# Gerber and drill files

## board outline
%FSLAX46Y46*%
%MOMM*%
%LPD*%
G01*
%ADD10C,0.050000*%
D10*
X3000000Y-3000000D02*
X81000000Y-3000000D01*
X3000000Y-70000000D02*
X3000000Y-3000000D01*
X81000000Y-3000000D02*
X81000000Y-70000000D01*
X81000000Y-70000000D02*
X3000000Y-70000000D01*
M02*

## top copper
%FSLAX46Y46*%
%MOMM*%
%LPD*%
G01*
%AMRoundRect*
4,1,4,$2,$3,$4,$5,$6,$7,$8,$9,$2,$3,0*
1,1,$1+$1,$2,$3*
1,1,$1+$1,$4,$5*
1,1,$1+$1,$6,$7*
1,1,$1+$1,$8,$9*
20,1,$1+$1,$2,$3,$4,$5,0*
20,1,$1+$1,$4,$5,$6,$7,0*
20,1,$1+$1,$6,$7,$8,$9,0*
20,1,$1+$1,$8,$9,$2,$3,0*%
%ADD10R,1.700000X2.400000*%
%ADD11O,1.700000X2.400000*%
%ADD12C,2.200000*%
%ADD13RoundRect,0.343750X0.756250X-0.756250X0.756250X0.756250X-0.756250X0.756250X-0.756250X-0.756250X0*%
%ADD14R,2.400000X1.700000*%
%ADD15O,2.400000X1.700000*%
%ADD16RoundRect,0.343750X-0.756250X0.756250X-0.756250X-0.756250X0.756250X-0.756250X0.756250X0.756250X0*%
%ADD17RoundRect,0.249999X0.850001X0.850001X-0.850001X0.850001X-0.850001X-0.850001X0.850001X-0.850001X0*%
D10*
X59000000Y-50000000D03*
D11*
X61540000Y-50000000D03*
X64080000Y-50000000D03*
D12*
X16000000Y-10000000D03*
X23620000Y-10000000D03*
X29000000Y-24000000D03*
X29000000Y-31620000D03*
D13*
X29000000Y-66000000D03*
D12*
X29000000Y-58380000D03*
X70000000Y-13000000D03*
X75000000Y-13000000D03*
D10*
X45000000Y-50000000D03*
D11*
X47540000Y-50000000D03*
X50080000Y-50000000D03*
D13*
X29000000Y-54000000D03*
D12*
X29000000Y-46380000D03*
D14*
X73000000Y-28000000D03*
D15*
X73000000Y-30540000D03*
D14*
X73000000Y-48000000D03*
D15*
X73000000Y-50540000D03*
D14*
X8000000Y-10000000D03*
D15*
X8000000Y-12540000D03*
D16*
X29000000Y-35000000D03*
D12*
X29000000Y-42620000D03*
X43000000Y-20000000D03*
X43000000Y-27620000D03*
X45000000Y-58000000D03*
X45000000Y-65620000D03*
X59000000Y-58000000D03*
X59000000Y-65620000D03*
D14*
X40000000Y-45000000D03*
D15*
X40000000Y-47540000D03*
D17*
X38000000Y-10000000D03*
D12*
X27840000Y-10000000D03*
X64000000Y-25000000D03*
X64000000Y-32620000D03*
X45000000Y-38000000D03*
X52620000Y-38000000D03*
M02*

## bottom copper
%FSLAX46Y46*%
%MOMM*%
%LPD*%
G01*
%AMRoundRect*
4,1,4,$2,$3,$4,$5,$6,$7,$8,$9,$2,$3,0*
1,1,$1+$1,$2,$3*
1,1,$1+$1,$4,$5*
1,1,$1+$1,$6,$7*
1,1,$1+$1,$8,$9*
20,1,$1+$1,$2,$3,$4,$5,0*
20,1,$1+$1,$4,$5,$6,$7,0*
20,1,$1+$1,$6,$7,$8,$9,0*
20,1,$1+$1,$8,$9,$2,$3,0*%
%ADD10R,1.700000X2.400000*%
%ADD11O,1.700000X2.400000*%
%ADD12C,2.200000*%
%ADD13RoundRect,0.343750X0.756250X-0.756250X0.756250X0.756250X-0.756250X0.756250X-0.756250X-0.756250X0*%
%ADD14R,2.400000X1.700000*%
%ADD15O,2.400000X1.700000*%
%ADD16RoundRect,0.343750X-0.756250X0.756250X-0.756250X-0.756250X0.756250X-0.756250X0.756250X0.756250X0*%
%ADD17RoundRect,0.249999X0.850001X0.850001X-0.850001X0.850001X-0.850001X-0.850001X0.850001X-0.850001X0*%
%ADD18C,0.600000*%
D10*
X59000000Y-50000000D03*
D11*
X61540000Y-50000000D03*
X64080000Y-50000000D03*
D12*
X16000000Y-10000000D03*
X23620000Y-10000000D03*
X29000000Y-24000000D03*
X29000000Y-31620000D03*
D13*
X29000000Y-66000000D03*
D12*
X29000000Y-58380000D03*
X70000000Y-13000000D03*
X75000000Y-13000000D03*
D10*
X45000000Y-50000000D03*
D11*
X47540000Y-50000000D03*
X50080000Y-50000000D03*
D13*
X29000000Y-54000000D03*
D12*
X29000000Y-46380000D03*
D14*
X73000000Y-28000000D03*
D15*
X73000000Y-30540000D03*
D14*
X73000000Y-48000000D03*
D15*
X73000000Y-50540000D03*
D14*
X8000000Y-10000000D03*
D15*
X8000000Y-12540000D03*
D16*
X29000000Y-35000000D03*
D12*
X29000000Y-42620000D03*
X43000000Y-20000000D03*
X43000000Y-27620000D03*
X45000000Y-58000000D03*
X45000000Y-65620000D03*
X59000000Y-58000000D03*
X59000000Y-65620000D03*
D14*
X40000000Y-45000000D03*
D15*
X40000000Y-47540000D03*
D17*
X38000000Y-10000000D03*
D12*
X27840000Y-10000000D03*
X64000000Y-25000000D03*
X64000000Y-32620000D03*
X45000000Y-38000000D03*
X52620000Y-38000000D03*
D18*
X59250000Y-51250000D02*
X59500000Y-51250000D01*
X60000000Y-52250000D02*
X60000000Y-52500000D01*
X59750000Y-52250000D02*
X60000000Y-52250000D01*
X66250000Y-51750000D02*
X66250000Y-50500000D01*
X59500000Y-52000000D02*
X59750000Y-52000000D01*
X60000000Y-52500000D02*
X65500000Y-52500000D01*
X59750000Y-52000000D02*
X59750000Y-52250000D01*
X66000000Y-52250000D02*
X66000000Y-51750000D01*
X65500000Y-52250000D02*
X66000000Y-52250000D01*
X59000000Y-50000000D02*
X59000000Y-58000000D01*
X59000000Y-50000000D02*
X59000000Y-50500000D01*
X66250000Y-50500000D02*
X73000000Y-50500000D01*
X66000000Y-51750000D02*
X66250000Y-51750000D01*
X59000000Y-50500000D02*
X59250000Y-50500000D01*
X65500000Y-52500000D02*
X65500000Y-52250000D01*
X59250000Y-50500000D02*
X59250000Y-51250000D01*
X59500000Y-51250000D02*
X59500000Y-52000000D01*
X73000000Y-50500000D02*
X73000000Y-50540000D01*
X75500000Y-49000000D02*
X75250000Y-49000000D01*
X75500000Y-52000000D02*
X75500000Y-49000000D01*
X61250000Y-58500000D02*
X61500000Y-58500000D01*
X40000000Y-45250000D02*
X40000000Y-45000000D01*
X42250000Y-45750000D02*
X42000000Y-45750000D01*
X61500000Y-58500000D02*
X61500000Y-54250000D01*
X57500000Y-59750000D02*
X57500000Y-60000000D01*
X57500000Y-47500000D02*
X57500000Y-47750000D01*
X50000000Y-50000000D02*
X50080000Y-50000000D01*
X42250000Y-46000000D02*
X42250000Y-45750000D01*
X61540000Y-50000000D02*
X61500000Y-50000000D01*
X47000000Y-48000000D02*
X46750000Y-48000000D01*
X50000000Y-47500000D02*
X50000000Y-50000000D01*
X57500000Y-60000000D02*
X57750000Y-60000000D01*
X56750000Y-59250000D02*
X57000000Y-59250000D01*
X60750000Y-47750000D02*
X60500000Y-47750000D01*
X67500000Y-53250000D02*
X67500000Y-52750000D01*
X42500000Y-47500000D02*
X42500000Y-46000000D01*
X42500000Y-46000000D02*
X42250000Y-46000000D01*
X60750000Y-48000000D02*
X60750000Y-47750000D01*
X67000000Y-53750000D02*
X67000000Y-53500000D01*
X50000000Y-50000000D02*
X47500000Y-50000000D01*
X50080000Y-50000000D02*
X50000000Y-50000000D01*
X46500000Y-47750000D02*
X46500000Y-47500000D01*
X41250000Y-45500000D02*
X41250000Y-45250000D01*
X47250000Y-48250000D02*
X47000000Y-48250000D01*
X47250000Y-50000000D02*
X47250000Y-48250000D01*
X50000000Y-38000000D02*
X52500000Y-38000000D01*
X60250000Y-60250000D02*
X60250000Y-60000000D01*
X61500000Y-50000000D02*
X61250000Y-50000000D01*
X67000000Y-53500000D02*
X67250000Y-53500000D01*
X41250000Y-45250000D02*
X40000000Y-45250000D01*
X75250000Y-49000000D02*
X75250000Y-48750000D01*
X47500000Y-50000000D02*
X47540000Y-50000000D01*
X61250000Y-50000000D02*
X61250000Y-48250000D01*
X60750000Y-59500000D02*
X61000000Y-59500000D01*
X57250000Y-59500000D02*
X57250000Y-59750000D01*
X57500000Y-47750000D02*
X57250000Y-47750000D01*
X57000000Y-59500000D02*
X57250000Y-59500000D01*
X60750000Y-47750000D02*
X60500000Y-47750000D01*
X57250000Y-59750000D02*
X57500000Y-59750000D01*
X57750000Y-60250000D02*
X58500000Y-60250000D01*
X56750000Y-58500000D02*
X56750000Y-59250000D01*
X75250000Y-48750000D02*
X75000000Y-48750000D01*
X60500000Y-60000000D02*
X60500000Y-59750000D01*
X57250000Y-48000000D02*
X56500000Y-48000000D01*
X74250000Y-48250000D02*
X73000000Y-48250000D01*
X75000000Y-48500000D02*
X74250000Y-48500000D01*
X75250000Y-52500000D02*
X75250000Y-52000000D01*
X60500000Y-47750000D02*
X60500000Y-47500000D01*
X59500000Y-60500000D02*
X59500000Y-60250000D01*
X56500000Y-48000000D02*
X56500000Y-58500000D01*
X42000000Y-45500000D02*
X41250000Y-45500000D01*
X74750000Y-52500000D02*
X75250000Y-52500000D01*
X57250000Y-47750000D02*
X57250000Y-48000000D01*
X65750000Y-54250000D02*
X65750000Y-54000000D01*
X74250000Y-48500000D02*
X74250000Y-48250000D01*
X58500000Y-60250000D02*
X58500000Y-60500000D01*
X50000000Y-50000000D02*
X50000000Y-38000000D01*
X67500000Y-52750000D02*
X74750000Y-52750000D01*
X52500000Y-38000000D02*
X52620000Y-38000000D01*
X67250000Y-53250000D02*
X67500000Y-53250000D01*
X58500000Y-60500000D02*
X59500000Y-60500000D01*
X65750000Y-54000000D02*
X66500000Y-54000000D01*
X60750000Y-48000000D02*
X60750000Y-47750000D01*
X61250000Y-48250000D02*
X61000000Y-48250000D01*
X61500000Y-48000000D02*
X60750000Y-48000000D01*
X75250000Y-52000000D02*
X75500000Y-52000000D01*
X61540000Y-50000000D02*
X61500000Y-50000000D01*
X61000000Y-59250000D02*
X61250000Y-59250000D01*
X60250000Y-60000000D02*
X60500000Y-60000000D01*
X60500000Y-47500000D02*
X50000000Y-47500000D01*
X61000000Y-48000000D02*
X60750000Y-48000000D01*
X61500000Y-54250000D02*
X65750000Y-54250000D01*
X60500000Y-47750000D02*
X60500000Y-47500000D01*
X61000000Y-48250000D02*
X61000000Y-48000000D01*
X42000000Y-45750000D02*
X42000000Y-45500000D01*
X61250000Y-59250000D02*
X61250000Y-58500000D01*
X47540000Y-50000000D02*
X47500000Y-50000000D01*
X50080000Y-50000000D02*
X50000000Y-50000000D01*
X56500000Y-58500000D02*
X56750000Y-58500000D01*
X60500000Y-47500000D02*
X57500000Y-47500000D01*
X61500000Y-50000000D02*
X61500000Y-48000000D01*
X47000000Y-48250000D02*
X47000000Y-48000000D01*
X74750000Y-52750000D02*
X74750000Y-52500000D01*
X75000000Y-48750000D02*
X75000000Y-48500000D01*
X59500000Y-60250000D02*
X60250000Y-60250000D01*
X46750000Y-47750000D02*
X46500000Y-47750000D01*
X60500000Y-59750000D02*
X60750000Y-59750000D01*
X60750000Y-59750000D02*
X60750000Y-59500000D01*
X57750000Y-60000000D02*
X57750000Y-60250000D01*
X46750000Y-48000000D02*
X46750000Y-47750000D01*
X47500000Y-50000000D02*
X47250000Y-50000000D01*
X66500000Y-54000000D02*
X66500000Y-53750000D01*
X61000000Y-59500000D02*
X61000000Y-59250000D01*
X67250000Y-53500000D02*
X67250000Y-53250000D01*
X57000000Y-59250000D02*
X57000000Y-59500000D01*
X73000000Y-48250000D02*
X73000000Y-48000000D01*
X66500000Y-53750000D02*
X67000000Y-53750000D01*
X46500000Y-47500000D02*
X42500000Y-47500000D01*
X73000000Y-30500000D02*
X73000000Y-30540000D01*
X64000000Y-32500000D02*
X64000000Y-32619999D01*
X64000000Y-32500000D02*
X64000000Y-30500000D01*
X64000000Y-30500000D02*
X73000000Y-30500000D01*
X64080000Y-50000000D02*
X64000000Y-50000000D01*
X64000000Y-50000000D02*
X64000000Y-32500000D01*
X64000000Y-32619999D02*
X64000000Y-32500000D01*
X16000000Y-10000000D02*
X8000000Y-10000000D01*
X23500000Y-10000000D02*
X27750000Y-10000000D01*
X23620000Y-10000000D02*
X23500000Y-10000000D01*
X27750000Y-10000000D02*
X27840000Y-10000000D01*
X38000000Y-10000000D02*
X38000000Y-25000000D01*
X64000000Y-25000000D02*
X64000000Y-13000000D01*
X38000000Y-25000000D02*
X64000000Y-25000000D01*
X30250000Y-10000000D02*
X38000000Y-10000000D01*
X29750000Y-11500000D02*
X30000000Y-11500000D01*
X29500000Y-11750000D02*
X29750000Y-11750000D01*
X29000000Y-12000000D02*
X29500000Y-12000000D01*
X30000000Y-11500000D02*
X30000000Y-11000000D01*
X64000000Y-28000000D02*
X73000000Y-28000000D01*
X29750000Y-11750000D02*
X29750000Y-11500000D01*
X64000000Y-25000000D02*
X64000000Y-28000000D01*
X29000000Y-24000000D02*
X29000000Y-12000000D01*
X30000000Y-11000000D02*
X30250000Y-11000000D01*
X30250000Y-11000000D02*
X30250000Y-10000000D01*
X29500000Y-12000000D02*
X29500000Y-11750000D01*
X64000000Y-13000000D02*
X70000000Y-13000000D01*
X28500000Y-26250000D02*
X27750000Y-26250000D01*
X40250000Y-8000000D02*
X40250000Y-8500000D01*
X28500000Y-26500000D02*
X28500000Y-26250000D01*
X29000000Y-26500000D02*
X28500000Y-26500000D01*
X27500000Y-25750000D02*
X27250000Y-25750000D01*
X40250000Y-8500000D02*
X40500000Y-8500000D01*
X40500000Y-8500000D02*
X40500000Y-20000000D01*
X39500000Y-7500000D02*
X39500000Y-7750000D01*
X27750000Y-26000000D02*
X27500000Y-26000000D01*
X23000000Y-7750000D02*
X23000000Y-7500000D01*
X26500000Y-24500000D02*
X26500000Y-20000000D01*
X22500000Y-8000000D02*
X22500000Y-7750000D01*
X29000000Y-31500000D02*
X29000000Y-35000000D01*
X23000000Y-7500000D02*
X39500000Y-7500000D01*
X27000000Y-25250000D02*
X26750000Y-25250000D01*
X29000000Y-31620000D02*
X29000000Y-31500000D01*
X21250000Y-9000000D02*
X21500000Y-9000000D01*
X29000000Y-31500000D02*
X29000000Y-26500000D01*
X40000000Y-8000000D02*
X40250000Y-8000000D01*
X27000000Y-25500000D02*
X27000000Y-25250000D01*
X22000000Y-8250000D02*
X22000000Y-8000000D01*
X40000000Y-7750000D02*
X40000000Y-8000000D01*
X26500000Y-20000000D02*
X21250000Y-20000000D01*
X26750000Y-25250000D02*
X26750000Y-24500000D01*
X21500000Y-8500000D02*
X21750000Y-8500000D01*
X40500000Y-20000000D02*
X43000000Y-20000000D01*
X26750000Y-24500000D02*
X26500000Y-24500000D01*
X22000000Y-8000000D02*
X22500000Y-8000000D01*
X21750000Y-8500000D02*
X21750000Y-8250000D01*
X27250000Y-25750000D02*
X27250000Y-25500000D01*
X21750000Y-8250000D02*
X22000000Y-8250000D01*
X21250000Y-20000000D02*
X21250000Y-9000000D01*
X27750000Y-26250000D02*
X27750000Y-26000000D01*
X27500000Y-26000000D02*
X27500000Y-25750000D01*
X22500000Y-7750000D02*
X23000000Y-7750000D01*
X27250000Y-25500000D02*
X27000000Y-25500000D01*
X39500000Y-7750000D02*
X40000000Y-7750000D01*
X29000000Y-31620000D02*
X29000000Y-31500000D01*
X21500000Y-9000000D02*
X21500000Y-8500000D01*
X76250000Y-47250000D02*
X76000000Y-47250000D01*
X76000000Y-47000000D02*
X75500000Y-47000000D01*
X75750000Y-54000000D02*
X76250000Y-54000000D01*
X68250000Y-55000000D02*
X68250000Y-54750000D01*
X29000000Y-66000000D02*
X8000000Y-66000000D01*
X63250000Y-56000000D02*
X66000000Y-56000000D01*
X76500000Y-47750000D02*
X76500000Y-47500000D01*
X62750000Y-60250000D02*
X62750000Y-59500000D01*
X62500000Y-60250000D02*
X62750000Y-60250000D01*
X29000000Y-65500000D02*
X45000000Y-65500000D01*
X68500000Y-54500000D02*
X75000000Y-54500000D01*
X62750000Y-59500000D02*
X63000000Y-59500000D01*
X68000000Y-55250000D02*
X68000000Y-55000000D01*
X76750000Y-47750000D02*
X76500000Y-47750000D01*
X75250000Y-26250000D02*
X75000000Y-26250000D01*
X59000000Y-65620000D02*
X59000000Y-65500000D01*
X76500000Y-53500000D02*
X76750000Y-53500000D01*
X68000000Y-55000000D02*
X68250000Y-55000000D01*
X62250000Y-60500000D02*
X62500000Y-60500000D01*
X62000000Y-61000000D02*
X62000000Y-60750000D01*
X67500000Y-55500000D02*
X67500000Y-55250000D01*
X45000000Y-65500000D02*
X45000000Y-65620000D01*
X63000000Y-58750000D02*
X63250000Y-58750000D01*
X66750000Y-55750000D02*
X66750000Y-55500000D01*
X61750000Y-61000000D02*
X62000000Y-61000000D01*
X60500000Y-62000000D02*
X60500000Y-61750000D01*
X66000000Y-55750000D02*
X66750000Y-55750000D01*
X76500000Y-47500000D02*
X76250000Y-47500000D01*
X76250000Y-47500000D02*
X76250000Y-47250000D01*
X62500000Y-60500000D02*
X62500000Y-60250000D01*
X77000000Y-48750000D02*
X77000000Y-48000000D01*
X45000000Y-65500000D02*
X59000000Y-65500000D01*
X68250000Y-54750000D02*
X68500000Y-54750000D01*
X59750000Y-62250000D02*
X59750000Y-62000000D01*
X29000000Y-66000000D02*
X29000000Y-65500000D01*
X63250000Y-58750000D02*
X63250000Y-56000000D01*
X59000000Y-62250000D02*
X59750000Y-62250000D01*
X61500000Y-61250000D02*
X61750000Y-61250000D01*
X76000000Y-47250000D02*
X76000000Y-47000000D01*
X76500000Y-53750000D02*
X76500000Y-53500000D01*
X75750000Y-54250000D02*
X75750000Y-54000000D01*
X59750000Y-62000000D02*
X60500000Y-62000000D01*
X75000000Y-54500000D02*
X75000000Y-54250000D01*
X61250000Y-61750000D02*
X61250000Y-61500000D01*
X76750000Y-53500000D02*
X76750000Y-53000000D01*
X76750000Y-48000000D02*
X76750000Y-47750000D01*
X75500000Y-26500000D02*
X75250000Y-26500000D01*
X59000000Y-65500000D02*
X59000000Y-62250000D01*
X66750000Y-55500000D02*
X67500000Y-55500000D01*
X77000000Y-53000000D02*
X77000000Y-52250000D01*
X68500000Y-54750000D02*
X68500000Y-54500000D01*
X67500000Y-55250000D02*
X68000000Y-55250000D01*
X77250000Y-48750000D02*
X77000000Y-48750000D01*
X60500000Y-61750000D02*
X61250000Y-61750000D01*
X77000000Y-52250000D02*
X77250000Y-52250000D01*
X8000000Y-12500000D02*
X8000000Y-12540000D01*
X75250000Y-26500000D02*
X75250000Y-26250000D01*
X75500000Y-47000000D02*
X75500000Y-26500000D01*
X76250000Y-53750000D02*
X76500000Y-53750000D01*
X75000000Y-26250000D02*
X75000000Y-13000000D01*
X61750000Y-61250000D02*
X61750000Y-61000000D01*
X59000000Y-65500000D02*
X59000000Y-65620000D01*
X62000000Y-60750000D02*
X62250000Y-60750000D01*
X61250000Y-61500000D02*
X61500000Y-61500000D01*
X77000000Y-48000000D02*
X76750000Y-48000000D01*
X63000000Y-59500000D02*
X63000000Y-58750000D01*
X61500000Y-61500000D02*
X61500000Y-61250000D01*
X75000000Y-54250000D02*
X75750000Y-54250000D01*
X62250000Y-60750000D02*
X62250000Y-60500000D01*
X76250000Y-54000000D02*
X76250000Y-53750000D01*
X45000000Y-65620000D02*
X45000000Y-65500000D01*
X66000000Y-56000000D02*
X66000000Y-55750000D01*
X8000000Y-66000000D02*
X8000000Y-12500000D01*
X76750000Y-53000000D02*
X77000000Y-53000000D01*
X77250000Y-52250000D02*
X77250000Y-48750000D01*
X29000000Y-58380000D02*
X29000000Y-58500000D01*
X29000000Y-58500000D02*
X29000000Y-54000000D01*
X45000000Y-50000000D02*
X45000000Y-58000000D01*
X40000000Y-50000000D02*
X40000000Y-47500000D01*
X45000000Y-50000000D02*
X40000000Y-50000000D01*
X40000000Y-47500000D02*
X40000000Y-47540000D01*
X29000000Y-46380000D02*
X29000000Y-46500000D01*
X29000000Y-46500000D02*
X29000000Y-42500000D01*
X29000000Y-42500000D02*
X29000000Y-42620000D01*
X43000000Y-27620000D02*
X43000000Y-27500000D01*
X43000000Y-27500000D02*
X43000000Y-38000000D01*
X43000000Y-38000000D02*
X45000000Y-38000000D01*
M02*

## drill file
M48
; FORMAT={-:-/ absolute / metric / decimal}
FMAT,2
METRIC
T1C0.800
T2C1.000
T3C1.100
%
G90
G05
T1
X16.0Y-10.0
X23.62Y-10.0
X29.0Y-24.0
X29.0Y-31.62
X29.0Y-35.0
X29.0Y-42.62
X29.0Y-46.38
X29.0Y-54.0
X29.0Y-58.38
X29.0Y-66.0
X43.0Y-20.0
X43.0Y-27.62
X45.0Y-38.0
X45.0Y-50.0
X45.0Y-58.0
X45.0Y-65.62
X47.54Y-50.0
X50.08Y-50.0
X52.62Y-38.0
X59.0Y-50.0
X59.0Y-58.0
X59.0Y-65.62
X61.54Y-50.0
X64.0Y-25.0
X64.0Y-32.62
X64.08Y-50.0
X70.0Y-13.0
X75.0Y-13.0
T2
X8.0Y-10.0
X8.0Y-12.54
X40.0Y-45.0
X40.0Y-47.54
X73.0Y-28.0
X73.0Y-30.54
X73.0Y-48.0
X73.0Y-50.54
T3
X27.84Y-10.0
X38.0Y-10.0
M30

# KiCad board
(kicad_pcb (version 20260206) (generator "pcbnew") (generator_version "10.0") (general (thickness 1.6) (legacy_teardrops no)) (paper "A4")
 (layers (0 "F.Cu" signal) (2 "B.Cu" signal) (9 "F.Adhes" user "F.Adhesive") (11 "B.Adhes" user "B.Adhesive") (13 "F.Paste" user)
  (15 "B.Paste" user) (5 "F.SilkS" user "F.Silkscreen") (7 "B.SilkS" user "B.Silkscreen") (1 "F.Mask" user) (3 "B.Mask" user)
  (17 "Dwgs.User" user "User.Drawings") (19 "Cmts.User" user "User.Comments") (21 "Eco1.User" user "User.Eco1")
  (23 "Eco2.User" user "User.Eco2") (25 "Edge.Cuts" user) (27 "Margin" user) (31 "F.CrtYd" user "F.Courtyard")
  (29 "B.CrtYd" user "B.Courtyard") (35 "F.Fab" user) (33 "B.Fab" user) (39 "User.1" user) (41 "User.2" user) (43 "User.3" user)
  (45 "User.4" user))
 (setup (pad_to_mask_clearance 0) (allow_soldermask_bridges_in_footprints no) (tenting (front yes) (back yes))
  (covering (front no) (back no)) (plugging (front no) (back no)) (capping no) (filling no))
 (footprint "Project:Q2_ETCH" (layer "F.Cu") (at 59 50)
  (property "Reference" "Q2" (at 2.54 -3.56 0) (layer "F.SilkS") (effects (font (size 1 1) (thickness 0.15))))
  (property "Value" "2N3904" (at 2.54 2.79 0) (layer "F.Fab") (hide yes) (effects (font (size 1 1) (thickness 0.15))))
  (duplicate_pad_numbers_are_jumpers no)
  (pad "1" thru_hole rect (at 0 0) (size 1.7 2.4) (drill 0.8) (layers "*.Cu" "*.Mask") (remove_unused_layers no) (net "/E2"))
  (pad "2" thru_hole oval (at 2.54 0) (size 1.7 2.4) (drill 0.8) (layers "*.Cu" "*.Mask") (remove_unused_layers no) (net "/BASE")
   (thermal_bridge_angle 45))
  (pad "3" thru_hole oval (at 5.08 0) (size 1.7 2.4) (drill 0.8) (layers "*.Cu" "*.Mask") (remove_unused_layers no) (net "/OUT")
   (thermal_bridge_angle 45)))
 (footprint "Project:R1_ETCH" (layer "F.Cu") (at 16 10)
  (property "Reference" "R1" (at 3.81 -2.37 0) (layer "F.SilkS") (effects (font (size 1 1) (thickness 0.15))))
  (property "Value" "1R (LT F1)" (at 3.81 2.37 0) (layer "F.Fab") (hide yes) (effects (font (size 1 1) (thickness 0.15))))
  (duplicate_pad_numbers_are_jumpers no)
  (pad "1" thru_hole circle (at 0 0) (size 2.2 2.2) (drill 0.8) (layers "*.Cu" "*.Mask") (remove_unused_layers no) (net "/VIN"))
  (pad "2" thru_hole circle (at 7.62 0) (size 2.2 2.2) (drill 0.8) (layers "*.Cu" "*.Mask") (remove_unused_layers no) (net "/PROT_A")))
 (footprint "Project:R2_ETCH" (layer "F.Cu") (at 29 24 -90)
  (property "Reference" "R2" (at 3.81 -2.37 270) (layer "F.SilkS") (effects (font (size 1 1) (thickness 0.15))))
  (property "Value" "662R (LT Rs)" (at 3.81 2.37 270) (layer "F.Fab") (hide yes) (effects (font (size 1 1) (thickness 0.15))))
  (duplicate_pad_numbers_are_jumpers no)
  (pad "1" thru_hole circle (at 0 0 270) (size 2.2 2.2) (drill 0.8) (layers "*.Cu" "*.Mask") (remove_unused_layers no) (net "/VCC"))
  (pad "2" thru_hole circle (at 7.62 0 270) (size 2.2 2.2) (drill 0.8) (layers "*.Cu" "*.Mask") (remove_unused_layers no) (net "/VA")))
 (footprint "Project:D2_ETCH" (layer "F.Cu") (at 29 66 90)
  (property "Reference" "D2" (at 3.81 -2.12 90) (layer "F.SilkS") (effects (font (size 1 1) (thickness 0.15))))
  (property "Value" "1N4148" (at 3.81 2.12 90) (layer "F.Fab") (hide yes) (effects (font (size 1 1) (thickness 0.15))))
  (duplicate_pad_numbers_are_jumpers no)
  (pad "1" thru_hole roundrect (at 0 0 90) (size 2.2 2.2) (drill 0.8) (layers "*.Cu" "*.Mask") (remove_unused_layers no)
   (roundrect_rratio 0.15625) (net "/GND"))
  (pad "2" thru_hole circle (at 7.62 0 90) (size 2.2 2.2) (drill 0.8) (layers "*.Cu" "*.Mask") (remove_unused_layers no) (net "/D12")))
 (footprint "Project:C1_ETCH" (layer "F.Cu") (at 70 13)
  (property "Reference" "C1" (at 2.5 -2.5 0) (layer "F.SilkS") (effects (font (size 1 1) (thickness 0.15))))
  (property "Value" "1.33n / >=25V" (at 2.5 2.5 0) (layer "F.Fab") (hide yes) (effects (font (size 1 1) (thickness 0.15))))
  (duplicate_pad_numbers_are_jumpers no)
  (pad "1" thru_hole circle (at 0 0) (size 2.2 2.2) (drill 0.8) (layers "*.Cu" "*.Mask") (remove_unused_layers no) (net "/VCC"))
  (pad "2" thru_hole circle (at 5 0) (size 2.2 2.2) (drill 0.8) (layers "*.Cu" "*.Mask") (remove_unused_layers no) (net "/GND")))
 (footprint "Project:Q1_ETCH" (layer "F.Cu") (at 45 50)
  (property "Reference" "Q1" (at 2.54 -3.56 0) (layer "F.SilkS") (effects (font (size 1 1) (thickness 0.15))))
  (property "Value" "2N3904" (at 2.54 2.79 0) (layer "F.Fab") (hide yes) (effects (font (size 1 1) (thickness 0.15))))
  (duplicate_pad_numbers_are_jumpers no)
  (pad "1" thru_hole rect (at 0 0) (size 1.7 2.4) (drill 0.8) (layers "*.Cu" "*.Mask") (remove_unused_layers no) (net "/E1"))
  (pad "2" thru_hole oval (at 2.54 0) (size 1.7 2.4) (drill 0.8) (layers "*.Cu" "*.Mask") (remove_unused_layers no) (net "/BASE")
   (thermal_bridge_angle 45))
  (pad "3" thru_hole oval (at 5.08 0) (size 1.7 2.4) (drill 0.8) (layers "*.Cu" "*.Mask") (remove_unused_layers no) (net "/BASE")
   (thermal_bridge_angle 45)))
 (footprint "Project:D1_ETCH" (layer "F.Cu") (at 29 54 90)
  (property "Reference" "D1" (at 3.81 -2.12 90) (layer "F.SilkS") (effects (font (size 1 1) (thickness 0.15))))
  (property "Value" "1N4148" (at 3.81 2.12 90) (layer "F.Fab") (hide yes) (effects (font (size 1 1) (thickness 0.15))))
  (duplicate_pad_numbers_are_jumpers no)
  (pad "1" thru_hole roundrect (at 0 0 90) (size 2.2 2.2) (drill 0.8) (layers "*.Cu" "*.Mask") (remove_unused_layers no)
   (roundrect_rratio 0.15625) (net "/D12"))
  (pad "2" thru_hole circle (at 7.62 0 90) (size 2.2 2.2) (drill 0.8) (layers "*.Cu" "*.Mask") (remove_unused_layers no) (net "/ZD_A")))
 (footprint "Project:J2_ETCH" (layer "F.Cu") (at 73 28)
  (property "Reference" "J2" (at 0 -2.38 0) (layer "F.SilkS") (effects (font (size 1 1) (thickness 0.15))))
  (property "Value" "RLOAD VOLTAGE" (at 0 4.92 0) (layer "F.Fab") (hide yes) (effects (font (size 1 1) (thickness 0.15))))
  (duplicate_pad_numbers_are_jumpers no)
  (pad "1" thru_hole rect (at 0 0) (size 2.4 1.7) (drill 1) (layers "*.Cu" "*.Mask") (remove_unused_layers no) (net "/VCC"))
  (pad "2" thru_hole oval (at 0 2.54) (size 2.4 1.7) (drill 1) (layers "*.Cu" "*.Mask") (remove_unused_layers no) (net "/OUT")
   (thermal_bridge_angle 45)))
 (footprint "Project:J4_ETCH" (layer "F.Cu") (at 73 48)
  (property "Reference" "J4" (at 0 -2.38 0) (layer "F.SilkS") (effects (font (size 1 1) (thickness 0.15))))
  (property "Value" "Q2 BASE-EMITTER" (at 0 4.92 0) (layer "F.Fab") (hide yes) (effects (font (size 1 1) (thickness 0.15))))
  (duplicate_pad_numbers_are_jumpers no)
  (pad "1" thru_hole rect (at 0 0) (size 2.4 1.7) (drill 1) (layers "*.Cu" "*.Mask") (remove_unused_layers no) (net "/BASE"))
  (pad "2" thru_hole oval (at 0 2.54) (size 2.4 1.7) (drill 1) (layers "*.Cu" "*.Mask") (remove_unused_layers no) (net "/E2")
   (thermal_bridge_angle 45)))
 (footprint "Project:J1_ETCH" (layer "F.Cu") (at 8 10)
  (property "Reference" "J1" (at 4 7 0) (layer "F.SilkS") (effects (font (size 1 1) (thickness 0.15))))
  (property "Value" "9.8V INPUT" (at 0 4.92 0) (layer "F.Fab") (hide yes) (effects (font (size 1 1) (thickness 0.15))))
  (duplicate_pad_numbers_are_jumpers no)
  (pad "1" thru_hole rect (at 0 0) (size 2.4 1.7) (drill 1) (layers "*.Cu" "*.Mask") (remove_unused_layers no) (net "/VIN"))
  (pad "2" thru_hole oval (at 0 2.54) (size 2.4 1.7) (drill 1) (layers "*.Cu" "*.Mask") (remove_unused_layers no) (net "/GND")
   (thermal_bridge_angle 45)))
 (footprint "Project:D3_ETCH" (layer "F.Cu") (at 29 35 -90)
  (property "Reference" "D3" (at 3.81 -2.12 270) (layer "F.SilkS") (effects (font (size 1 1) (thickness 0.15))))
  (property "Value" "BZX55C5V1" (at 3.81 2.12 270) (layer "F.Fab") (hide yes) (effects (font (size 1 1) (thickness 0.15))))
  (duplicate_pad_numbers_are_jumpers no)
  (pad "1" thru_hole roundrect (at 0 0 270) (size 2.2 2.2) (drill 0.8) (layers "*.Cu" "*.Mask") (remove_unused_layers no)
   (roundrect_rratio 0.15625) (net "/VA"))
  (pad "2" thru_hole circle (at 7.62 0 270) (size 2.2 2.2) (drill 0.8) (layers "*.Cu" "*.Mask") (remove_unused_layers no) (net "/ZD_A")))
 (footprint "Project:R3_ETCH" (layer "F.Cu") (at 43 20 -90)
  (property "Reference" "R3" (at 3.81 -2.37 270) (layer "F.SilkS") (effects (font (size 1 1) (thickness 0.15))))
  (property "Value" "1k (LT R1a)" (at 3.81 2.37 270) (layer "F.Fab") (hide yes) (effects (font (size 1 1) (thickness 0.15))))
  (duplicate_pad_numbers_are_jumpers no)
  (pad "1" thru_hole circle (at 0 0 270) (size 2.2 2.2) (drill 0.8) (layers "*.Cu" "*.Mask") (remove_unused_layers no) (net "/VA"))
  (pad "2" thru_hole circle (at 7.62 0 270) (size 2.2 2.2) (drill 0.8) (layers "*.Cu" "*.Mask") (remove_unused_layers no) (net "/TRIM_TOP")))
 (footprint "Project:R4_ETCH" (layer "F.Cu") (at 45 58 -90)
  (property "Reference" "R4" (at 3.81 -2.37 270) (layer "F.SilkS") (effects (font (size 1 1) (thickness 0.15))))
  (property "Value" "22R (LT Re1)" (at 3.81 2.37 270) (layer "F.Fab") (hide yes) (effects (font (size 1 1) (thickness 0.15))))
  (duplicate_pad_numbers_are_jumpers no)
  (pad "1" thru_hole circle (at 0 0 270) (size 2.2 2.2) (drill 0.8) (layers "*.Cu" "*.Mask") (remove_unused_layers no) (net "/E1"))
  (pad "2" thru_hole circle (at 7.62 0 270) (size 2.2 2.2) (drill 0.8) (layers "*.Cu" "*.Mask") (remove_unused_layers no) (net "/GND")))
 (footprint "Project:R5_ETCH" (layer "F.Cu") (at 59 58 -90)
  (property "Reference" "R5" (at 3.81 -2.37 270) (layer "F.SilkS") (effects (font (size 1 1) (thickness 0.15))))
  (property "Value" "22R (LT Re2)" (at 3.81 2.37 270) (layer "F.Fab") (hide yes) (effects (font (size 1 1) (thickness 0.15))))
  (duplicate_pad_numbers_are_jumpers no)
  (pad "1" thru_hole circle (at 0 0 270) (size 2.2 2.2) (drill 0.8) (layers "*.Cu" "*.Mask") (remove_unused_layers no) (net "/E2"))
  (pad "2" thru_hole circle (at 7.62 0 270) (size 2.2 2.2) (drill 0.8) (layers "*.Cu" "*.Mask") (remove_unused_layers no) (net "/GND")))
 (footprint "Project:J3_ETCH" (layer "F.Cu") (at 40 45)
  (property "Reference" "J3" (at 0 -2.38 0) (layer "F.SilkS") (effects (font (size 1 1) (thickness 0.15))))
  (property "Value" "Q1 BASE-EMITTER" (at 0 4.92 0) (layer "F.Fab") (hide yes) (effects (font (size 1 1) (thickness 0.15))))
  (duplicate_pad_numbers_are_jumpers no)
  (pad "1" thru_hole rect (at 0 0) (size 2.4 1.7) (drill 1) (layers "*.Cu" "*.Mask") (remove_unused_layers no) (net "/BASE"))
  (pad "2" thru_hole oval (at 0 2.54) (size 2.4 1.7) (drill 1) (layers "*.Cu" "*.Mask") (remove_unused_layers no) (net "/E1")
   (thermal_bridge_angle 45)))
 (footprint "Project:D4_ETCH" (layer "F.Cu") (at 38 10 180)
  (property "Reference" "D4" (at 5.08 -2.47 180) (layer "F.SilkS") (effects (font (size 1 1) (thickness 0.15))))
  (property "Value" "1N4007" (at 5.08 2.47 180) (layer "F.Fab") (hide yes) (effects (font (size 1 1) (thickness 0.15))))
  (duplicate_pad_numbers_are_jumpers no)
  (pad "1" thru_hole roundrect (at 0 0 180) (size 2.2 2.2) (drill 1.1) (layers "*.Cu" "*.Mask") (remove_unused_layers no)
   (roundrect_rratio 0.113636) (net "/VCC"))
  (pad "2" thru_hole circle (at 10.16 0 180) (size 2.2 2.2) (drill 1.1) (layers "*.Cu" "*.Mask") (remove_unused_layers no) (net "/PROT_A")))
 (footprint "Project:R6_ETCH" (layer "F.Cu") (at 64 25 -90)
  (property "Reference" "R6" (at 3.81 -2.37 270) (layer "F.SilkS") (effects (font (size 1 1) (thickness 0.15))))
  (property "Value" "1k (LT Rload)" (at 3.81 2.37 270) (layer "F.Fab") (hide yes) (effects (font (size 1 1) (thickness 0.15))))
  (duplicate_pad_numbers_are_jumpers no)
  (pad "1" thru_hole circle (at 0 0 270) (size 2.2 2.2) (drill 0.8) (layers "*.Cu" "*.Mask") (remove_unused_layers no) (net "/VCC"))
  (pad "2" thru_hole circle (at 7.62 0 270) (size 2.2 2.2) (drill 0.8) (layers "*.Cu" "*.Mask") (remove_unused_layers no) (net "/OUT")))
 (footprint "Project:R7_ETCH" (layer "F.Cu") (at 45 38)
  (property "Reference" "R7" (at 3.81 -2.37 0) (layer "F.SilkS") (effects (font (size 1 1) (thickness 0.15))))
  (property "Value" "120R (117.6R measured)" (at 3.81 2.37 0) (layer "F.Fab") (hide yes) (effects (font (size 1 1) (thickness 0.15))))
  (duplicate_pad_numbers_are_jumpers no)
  (pad "1" thru_hole circle (at 0 0) (size 2.2 2.2) (drill 0.8) (layers "*.Cu" "*.Mask") (remove_unused_layers no) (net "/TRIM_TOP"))
  (pad "2" thru_hole circle (at 7.62 0) (size 2.2 2.2) (drill 0.8) (layers "*.Cu" "*.Mask") (remove_unused_layers no) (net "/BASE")))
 (gr_line (start 3 3) (end 81 3) (stroke (width 0.05) (type default)) (layer "Edge.Cuts"))
 (gr_line (start 3 70) (end 3 3) (stroke (width 0.05) (type default)) (layer "Edge.Cuts"))
 (gr_line (start 81 3) (end 81 70) (stroke (width 0.05) (type default)) (layer "Edge.Cuts"))
 (gr_line (start 81 70) (end 3 70) (stroke (width 0.05) (type default)) (layer "Edge.Cuts"))
 (segment (start 59.25 51.25) (end 59.5 51.25) (width 0.6) (layer "B.Cu") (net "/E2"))
 (segment (start 60 52.25) (end 60 52.5) (width 0.6) (layer "B.Cu") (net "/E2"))
 (segment (start 59.75 52.25) (end 60 52.25) (width 0.6) (layer "B.Cu") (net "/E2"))
 (segment (start 66.25 51.75) (end 66.25 50.5) (width 0.6) (layer "B.Cu") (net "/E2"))
 (segment (start 59.5 52) (end 59.75 52) (width 0.6) (layer "B.Cu") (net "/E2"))
 (segment (start 60 52.5) (end 65.5 52.5) (width 0.6) (layer "B.Cu") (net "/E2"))
 (segment (start 59.75 52) (end 59.75 52.25) (width 0.6) (layer "B.Cu") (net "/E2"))
 (segment (start 66 52.25) (end 66 51.75) (width 0.6) (layer "B.Cu") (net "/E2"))
 (segment (start 65.5 52.25) (end 66 52.25) (width 0.6) (layer "B.Cu") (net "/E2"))
 (segment (start 59 50) (end 59 58) (width 0.6) (layer "B.Cu") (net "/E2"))
 (segment (start 59 50) (end 59 50.5) (width 0.6) (layer "B.Cu") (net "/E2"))
 (segment (start 66.25 50.5) (end 73 50.5) (width 0.6) (layer "B.Cu") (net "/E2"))
 (segment (start 66 51.75) (end 66.25 51.75) (width 0.6) (layer "B.Cu") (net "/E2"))
 (segment (start 59 50.5) (end 59.25 50.5) (width 0.6) (layer "B.Cu") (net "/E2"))
 (segment (start 65.5 52.5) (end 65.5 52.25) (width 0.6) (layer "B.Cu") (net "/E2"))
 (segment (start 59.25 50.5) (end 59.25 51.25) (width 0.6) (layer "B.Cu") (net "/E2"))
 (segment (start 59.5 51.25) (end 59.5 52) (width 0.6) (layer "B.Cu") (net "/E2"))
 (segment (start 73 50.5) (end 73 50.54) (width 0.6) (layer "B.Cu") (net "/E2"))
 (segment (start 75.5 49) (end 75.25 49) (width 0.6) (layer "B.Cu") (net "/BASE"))
 (segment (start 75.5 52) (end 75.5 49) (width 0.6) (layer "B.Cu") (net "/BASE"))
 (segment (start 61.25 58.5) (end 61.5 58.5) (width 0.6) (layer "B.Cu") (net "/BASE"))
 (segment (start 40 45.25) (end 40 45) (width 0.6) (layer "B.Cu") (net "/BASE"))
 (segment (start 42.25 45.75) (end 42 45.75) (width 0.6) (layer "B.Cu") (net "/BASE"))
 (segment (start 61.5 58.5) (end 61.5 54.25) (width 0.6) (layer "B.Cu") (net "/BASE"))
 (segment (start 57.5 59.75) (end 57.5 60) (width 0.6) (layer "B.Cu") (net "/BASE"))
 (segment (start 57.5 47.5) (end 57.5 47.75) (width 0.6) (layer "B.Cu") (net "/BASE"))
 (segment (start 50 50) (end 50.08 50) (width 0.6) (layer "B.Cu") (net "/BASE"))
 (segment (start 42.25 46) (end 42.25 45.75) (width 0.6) (layer "B.Cu") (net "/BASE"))
 (segment (start 61.54 50) (end 61.5 50) (width 0.6) (layer "B.Cu") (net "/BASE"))
 (segment (start 47 48) (end 46.75 48) (width 0.6) (layer "B.Cu") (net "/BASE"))
 (segment (start 50 47.5) (end 50 50) (width 0.6) (layer "B.Cu") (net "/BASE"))
 (segment (start 57.5 60) (end 57.75 60) (width 0.6) (layer "B.Cu") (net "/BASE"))
 (segment (start 56.75 59.25) (end 57 59.25) (width 0.6) (layer "B.Cu") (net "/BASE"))
 (segment (start 60.75 47.75) (end 60.5 47.75) (width 0.6) (layer "B.Cu") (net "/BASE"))
 (segment (start 67.5 53.25) (end 67.5 52.75) (width 0.6) (layer "B.Cu") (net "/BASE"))
 (segment (start 42.5 47.5) (end 42.5 46) (width 0.6) (layer "B.Cu") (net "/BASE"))
 (segment (start 42.5 46) (end 42.25 46) (width 0.6) (layer "B.Cu") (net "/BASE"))
 (segment (start 60.75 48) (end 60.75 47.75) (width 0.6) (layer "B.Cu") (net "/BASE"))
 (segment (start 67 53.75) (end 67 53.5) (width 0.6) (layer "B.Cu") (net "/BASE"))
 (segment (start 50 50) (end 47.5 50) (width 0.6) (layer "B.Cu") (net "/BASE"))
 (segment (start 50.08 50) (end 50 50) (width 0.6) (layer "B.Cu") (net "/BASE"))
 (segment (start 46.5 47.75) (end 46.5 47.5) (width 0.6) (layer "B.Cu") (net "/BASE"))
 (segment (start 41.25 45.5) (end 41.25 45.25) (width 0.6) (layer "B.Cu") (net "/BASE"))
 (segment (start 47.25 48.25) (end 47 48.25) (width 0.6) (layer "B.Cu") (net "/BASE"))
 (segment (start 47.25 50) (end 47.25 48.25) (width 0.6) (layer "B.Cu") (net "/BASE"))
 (segment (start 50 38) (end 52.5 38) (width 0.6) (layer "B.Cu") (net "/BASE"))
 (segment (start 60.25 60.25) (end 60.25 60) (width 0.6) (layer "B.Cu") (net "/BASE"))
 (segment (start 61.5 50) (end 61.25 50) (width 0.6) (layer "B.Cu") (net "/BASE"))
 (segment (start 67 53.5) (end 67.25 53.5) (width 0.6) (layer "B.Cu") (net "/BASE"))
 (segment (start 41.25 45.25) (end 40 45.25) (width 0.6) (layer "B.Cu") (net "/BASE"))
 (segment (start 75.25 49) (end 75.25 48.75) (width 0.6) (layer "B.Cu") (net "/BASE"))
 (segment (start 47.5 50) (end 47.54 50) (width 0.6) (layer "B.Cu") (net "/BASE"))
 (segment (start 61.25 50) (end 61.25 48.25) (width 0.6) (layer "B.Cu") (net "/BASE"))
 (segment (start 60.75 59.5) (end 61 59.5) (width 0.6) (layer "B.Cu") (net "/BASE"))
 (segment (start 57.25 59.5) (end 57.25 59.75) (width 0.6) (layer "B.Cu") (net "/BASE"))
 (segment (start 57.5 47.75) (end 57.25 47.75) (width 0.6) (layer "B.Cu") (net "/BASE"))
 (segment (start 57 59.5) (end 57.25 59.5) (width 0.6) (layer "B.Cu") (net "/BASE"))
 (segment (start 60.75 47.75) (end 60.5 47.75) (width 0.6) (layer "B.Cu") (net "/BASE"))
 (segment (start 57.25 59.75) (end 57.5 59.75) (width 0.6) (layer "B.Cu") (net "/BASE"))
 (segment (start 57.75 60.25) (end 58.5 60.25) (width 0.6) (layer "B.Cu") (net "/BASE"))
 (segment (start 56.75 58.5) (end 56.75 59.25) (width 0.6) (layer "B.Cu") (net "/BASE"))
 (segment (start 75.25 48.75) (end 75 48.75) (width 0.6) (layer "B.Cu") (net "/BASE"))
 (segment (start 60.5 60) (end 60.5 59.75) (width 0.6) (layer "B.Cu") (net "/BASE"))
 (segment (start 57.25 48) (end 56.5 48) (width 0.6) (layer "B.Cu") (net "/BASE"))
 (segment (start 74.25 48.25) (end 73 48.25) (width 0.6) (layer "B.Cu") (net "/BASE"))
 (segment (start 75 48.5) (end 74.25 48.5) (width 0.6) (layer "B.Cu") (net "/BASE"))
 (segment (start 75.25 52.5) (end 75.25 52) (width 0.6) (layer "B.Cu") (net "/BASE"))
 (segment (start 60.5 47.75) (end 60.5 47.5) (width 0.6) (layer "B.Cu") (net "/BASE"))
 (segment (start 59.5 60.5) (end 59.5 60.25) (width 0.6) (layer "B.Cu") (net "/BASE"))
 (segment (start 56.5 48) (end 56.5 58.5) (width 0.6) (layer "B.Cu") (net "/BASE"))
 (segment (start 42 45.5) (end 41.25 45.5) (width 0.6) (layer "B.Cu") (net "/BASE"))
 (segment (start 74.75 52.5) (end 75.25 52.5) (width 0.6) (layer "B.Cu") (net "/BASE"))
 (segment (start 57.25 47.75) (end 57.25 48) (width 0.6) (layer "B.Cu") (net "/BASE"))
 (segment (start 65.75 54.25) (end 65.75 54) (width 0.6) (layer "B.Cu") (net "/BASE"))
 (segment (start 74.25 48.5) (end 74.25 48.25) (width 0.6) (layer "B.Cu") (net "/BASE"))
 (segment (start 58.5 60.25) (end 58.5 60.5) (width 0.6) (layer "B.Cu") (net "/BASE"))
 (segment (start 50 50) (end 50 38) (width 0.6) (layer "B.Cu") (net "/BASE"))
 (segment (start 67.5 52.75) (end 74.75 52.75) (width 0.6) (layer "B.Cu") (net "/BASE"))
 (segment (start 52.5 38) (end 52.62 38) (width 0.6) (layer "B.Cu") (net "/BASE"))
 (segment (start 67.25 53.25) (end 67.5 53.25) (width 0.6) (layer "B.Cu") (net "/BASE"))
 (segment (start 58.5 60.5) (end 59.5 60.5) (width 0.6) (layer "B.Cu") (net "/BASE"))
 (segment (start 65.75 54) (end 66.5 54) (width 0.6) (layer "B.Cu") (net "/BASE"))
 (segment (start 60.75 48) (end 60.75 47.75) (width 0.6) (layer "B.Cu") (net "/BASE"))
 (segment (start 61.25 48.25) (end 61 48.25) (width 0.6) (layer "B.Cu") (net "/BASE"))
 (segment (start 61.5 48) (end 60.75 48) (width 0.6) (layer "B.Cu") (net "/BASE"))
 (segment (start 75.25 52) (end 75.5 52) (width 0.6) (layer "B.Cu") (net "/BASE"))
 (segment (start 61.54 50) (end 61.5 50) (width 0.6) (layer "B.Cu") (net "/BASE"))
 (segment (start 61 59.25) (end 61.25 59.25) (width 0.6) (layer "B.Cu") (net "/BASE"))
 (segment (start 60.25 60) (end 60.5 60) (width 0.6) (layer "B.Cu") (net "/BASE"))
 (segment (start 60.5 47.5) (end 50 47.5) (width 0.6) (layer "B.Cu") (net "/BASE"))
 (segment (start 61 48) (end 60.75 48) (width 0.6) (layer "B.Cu") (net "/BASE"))
 (segment (start 61.5 54.25) (end 65.75 54.25) (width 0.6) (layer "B.Cu") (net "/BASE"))
 (segment (start 60.5 47.75) (end 60.5 47.5) (width 0.6) (layer "B.Cu") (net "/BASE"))
 (segment (start 61 48.25) (end 61 48) (width 0.6) (layer "B.Cu") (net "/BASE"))
 (segment (start 42 45.75) (end 42 45.5) (width 0.6) (layer "B.Cu") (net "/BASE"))
 (segment (start 61.25 59.25) (end 61.25 58.5) (width 0.6) (layer "B.Cu") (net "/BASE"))
 (segment (start 47.54 50) (end 47.5 50) (width 0.6) (layer "B.Cu") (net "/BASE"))
 (segment (start 50.08 50) (end 50 50) (width 0.6) (layer "B.Cu") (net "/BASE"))
 (segment (start 56.5 58.5) (end 56.75 58.5) (width 0.6) (layer "B.Cu") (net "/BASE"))
 (segment (start 60.5 47.5) (end 57.5 47.5) (width 0.6) (layer "B.Cu") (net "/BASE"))
 (segment (start 61.5 50) (end 61.5 48) (width 0.6) (layer "B.Cu") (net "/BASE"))
 (segment (start 47 48.25) (end 47 48) (width 0.6) (layer "B.Cu") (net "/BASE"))
 (segment (start 74.75 52.75) (end 74.75 52.5) (width 0.6) (layer "B.Cu") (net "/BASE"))
 (segment (start 75 48.75) (end 75 48.5) (width 0.6) (layer "B.Cu") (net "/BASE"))
 (segment (start 59.5 60.25) (end 60.25 60.25) (width 0.6) (layer "B.Cu") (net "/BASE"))
 (segment (start 46.75 47.75) (end 46.5 47.75) (width 0.6) (layer "B.Cu") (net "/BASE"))
 (segment (start 60.5 59.75) (end 60.75 59.75) (width 0.6) (layer "B.Cu") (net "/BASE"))
 (segment (start 60.75 59.75) (end 60.75 59.5) (width 0.6) (layer "B.Cu") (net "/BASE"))
 (segment (start 57.75 60) (end 57.75 60.25) (width 0.6) (layer "B.Cu") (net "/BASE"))
 (segment (start 46.75 48) (end 46.75 47.75) (width 0.6) (layer "B.Cu") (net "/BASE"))
 (segment (start 47.5 50) (end 47.25 50) (width 0.6) (layer "B.Cu") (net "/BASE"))
 (segment (start 66.5 54) (end 66.5 53.75) (width 0.6) (layer "B.Cu") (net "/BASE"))
 (segment (start 61 59.5) (end 61 59.25) (width 0.6) (layer "B.Cu") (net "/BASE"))
 (segment (start 67.25 53.5) (end 67.25 53.25) (width 0.6) (layer "B.Cu") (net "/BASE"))
 (segment (start 57 59.25) (end 57 59.5) (width 0.6) (layer "B.Cu") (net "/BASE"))
 (segment (start 73 48.25) (end 73 48) (width 0.6) (layer "B.Cu") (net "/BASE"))
 (segment (start 66.5 53.75) (end 67 53.75) (width 0.6) (layer "B.Cu") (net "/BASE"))
 (segment (start 46.5 47.5) (end 42.5 47.5) (width 0.6) (layer "B.Cu") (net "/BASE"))
 (segment (start 73 30.5) (end 73 30.54) (width 0.6) (layer "B.Cu") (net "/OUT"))
 (segment (start 64 32.5) (end 64 32.619999) (width 0.6) (layer "B.Cu") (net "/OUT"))
 (segment (start 64 32.5) (end 64 30.5) (width 0.6) (layer "B.Cu") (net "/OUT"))
 (segment (start 64 30.5) (end 73 30.5) (width 0.6) (layer "B.Cu") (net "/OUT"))
 (segment (start 64.08 50) (end 64 50) (width 0.6) (layer "B.Cu") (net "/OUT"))
 (segment (start 64 50) (end 64 32.5) (width 0.6) (layer "B.Cu") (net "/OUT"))
 (segment (start 64 32.619999) (end 64 32.5) (width 0.6) (layer "B.Cu") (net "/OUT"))
 (segment (start 16 10) (end 8 10) (width 0.6) (layer "B.Cu") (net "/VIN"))
 (segment (start 23.5 10) (end 27.75 10) (width 0.6) (layer "B.Cu") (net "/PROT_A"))
 (segment (start 23.62 10) (end 23.5 10) (width 0.6) (layer "B.Cu") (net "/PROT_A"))
 (segment (start 27.75 10) (end 27.84 10) (width 0.6) (layer "B.Cu") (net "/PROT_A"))
 (segment (start 38 10) (end 38 25) (width 0.6) (layer "B.Cu") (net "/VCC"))
 (segment (start 64 25) (end 64 13) (width 0.6) (layer "B.Cu") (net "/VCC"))
 (segment (start 38 25) (end 64 25) (width 0.6) (layer "B.Cu") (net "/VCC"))
 (segment (start 30.25 10) (end 38 10) (width 0.6) (layer "B.Cu") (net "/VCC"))
 (segment (start 29.75 11.5) (end 30 11.5) (width 0.6) (layer "B.Cu") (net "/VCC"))
 (segment (start 29.5 11.75) (end 29.75 11.75) (width 0.6) (layer "B.Cu") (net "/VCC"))
 (segment (start 29 12) (end 29.5 12) (width 0.6) (layer "B.Cu") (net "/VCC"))
 (segment (start 30 11.5) (end 30 11) (width 0.6) (layer "B.Cu") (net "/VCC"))
 (segment (start 64 28) (end 73 28) (width 0.6) (layer "B.Cu") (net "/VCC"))
 (segment (start 29.75 11.75) (end 29.75 11.5) (width 0.6) (layer "B.Cu") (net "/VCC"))
 (segment (start 64 25) (end 64 28) (width 0.6) (layer "B.Cu") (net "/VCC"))
 (segment (start 29 24) (end 29 12) (width 0.6) (layer "B.Cu") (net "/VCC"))
 (segment (start 30 11) (end 30.25 11) (width 0.6) (layer "B.Cu") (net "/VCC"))
 (segment (start 30.25 11) (end 30.25 10) (width 0.6) (layer "B.Cu") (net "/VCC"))
 (segment (start 29.5 12) (end 29.5 11.75) (width 0.6) (layer "B.Cu") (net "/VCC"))
 (segment (start 64 13) (end 70 13) (width 0.6) (layer "B.Cu") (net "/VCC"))
 (segment (start 28.5 26.25) (end 27.75 26.25) (width 0.6) (layer "B.Cu") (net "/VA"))
 (segment (start 40.25 8) (end 40.25 8.5) (width 0.6) (layer "B.Cu") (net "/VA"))
 (segment (start 28.5 26.5) (end 28.5 26.25) (width 0.6) (layer "B.Cu") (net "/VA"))
 (segment (start 29 26.5) (end 28.5 26.5) (width 0.6) (layer "B.Cu") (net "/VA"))
 (segment (start 27.5 25.75) (end 27.25 25.75) (width 0.6) (layer "B.Cu") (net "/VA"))
 (segment (start 40.25 8.5) (end 40.5 8.5) (width 0.6) (layer "B.Cu") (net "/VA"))
 (segment (start 40.5 8.5) (end 40.5 20) (width 0.6) (layer "B.Cu") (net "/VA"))
 (segment (start 39.5 7.5) (end 39.5 7.75) (width 0.6) (layer "B.Cu") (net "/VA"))
 (segment (start 27.75 26) (end 27.5 26) (width 0.6) (layer "B.Cu") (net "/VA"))
 (segment (start 23 7.75) (end 23 7.5) (width 0.6) (layer "B.Cu") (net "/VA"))
 (segment (start 26.5 24.5) (end 26.5 20) (width 0.6) (layer "B.Cu") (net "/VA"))
 (segment (start 22.5 8) (end 22.5 7.75) (width 0.6) (layer "B.Cu") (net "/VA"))
 (segment (start 29 31.5) (end 29 35) (width 0.6) (layer "B.Cu") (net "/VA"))
 (segment (start 23 7.5) (end 39.5 7.5) (width 0.6) (layer "B.Cu") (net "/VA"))
 (segment (start 27 25.25) (end 26.75 25.25) (width 0.6) (layer "B.Cu") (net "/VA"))
 (segment (start 29 31.62) (end 29 31.5) (width 0.6) (layer "B.Cu") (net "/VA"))
 (segment (start 21.25 9) (end 21.5 9) (width 0.6) (layer "B.Cu") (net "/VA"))
 (segment (start 29 31.5) (end 29 26.5) (width 0.6) (layer "B.Cu") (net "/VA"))
 (segment (start 40 8) (end 40.25 8) (width 0.6) (layer "B.Cu") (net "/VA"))
 (segment (start 27 25.5) (end 27 25.25) (width 0.6) (layer "B.Cu") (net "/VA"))
 (segment (start 22 8.25) (end 22 8) (width 0.6) (layer "B.Cu") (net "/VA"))
 (segment (start 40 7.75) (end 40 8) (width 0.6) (layer "B.Cu") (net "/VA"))
 (segment (start 26.5 20) (end 21.25 20) (width 0.6) (layer "B.Cu") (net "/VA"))
 (segment (start 26.75 25.25) (end 26.75 24.5) (width 0.6) (layer "B.Cu") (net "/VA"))
 (segment (start 21.5 8.5) (end 21.75 8.5) (width 0.6) (layer "B.Cu") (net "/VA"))
 (segment (start 40.5 20) (end 43 20) (width 0.6) (layer "B.Cu") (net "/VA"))
 (segment (start 26.75 24.5) (end 26.5 24.5) (width 0.6) (layer "B.Cu") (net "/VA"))
 (segment (start 22 8) (end 22.5 8) (width 0.6) (layer "B.Cu") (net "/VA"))
 (segment (start 21.75 8.5) (end 21.75 8.25) (width 0.6) (layer "B.Cu") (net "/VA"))
 (segment (start 27.25 25.75) (end 27.25 25.5) (width 0.6) (layer "B.Cu") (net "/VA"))
 (segment (start 21.75 8.25) (end 22 8.25) (width 0.6) (layer "B.Cu") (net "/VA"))
 (segment (start 21.25 20) (end 21.25 9) (width 0.6) (layer "B.Cu") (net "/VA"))
 (segment (start 27.75 26.25) (end 27.75 26) (width 0.6) (layer "B.Cu") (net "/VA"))
 (segment (start 27.5 26) (end 27.5 25.75) (width 0.6) (layer "B.Cu") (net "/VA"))
 (segment (start 22.5 7.75) (end 23 7.75) (width 0.6) (layer "B.Cu") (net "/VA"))
 (segment (start 27.25 25.5) (end 27 25.5) (width 0.6) (layer "B.Cu") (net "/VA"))
 (segment (start 39.5 7.75) (end 40 7.75) (width 0.6) (layer "B.Cu") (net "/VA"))
 (segment (start 29 31.62) (end 29 31.5) (width 0.6) (layer "B.Cu") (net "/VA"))
 (segment (start 21.5 9) (end 21.5 8.5) (width 0.6) (layer "B.Cu") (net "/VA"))
 (segment (start 76.25 47.25) (end 76 47.25) (width 0.6) (layer "B.Cu") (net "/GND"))
 (segment (start 76 47) (end 75.5 47) (width 0.6) (layer "B.Cu") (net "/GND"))
 (segment (start 75.75 54) (end 76.25 54) (width 0.6) (layer "B.Cu") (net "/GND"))
 (segment (start 68.25 55) (end 68.25 54.75) (width 0.6) (layer "B.Cu") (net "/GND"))
 (segment (start 29 66) (end 8 66) (width 0.6) (layer "B.Cu") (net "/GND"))
 (segment (start 63.25 56) (end 66 56) (width 0.6) (layer "B.Cu") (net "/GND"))
 (segment (start 76.5 47.75) (end 76.5 47.5) (width 0.6) (layer "B.Cu") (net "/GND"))
 (segment (start 62.75 60.25) (end 62.75 59.5) (width 0.6) (layer "B.Cu") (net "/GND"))
 (segment (start 62.5 60.25) (end 62.75 60.25) (width 0.6) (layer "B.Cu") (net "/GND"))
 (segment (start 29 65.5) (end 45 65.5) (width 0.6) (layer "B.Cu") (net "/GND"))
 (segment (start 68.5 54.5) (end 75 54.5) (width 0.6) (layer "B.Cu") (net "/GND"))
 (segment (start 62.75 59.5) (end 63 59.5) (width 0.6) (layer "B.Cu") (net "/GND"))
 (segment (start 68 55.25) (end 68 55) (width 0.6) (layer "B.Cu") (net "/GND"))
 (segment (start 76.75 47.75) (end 76.5 47.75) (width 0.6) (layer "B.Cu") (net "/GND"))
 (segment (start 75.25 26.25) (end 75 26.25) (width 0.6) (layer "B.Cu") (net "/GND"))
 (segment (start 59 65.62) (end 59 65.5) (width 0.6) (layer "B.Cu") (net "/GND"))
 (segment (start 76.5 53.5) (end 76.75 53.5) (width 0.6) (layer "B.Cu") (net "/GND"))
 (segment (start 68 55) (end 68.25 55) (width 0.6) (layer "B.Cu") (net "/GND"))
 (segment (start 62.25 60.5) (end 62.5 60.5) (width 0.6) (layer "B.Cu") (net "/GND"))
 (segment (start 62 61) (end 62 60.75) (width 0.6) (layer "B.Cu") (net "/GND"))
 (segment (start 67.5 55.5) (end 67.5 55.25) (width 0.6) (layer "B.Cu") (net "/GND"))
 (segment (start 45 65.5) (end 45 65.62) (width 0.6) (layer "B.Cu") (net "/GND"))
 (segment (start 63 58.75) (end 63.25 58.75) (width 0.6) (layer "B.Cu") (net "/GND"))
 (segment (start 66.75 55.75) (end 66.75 55.5) (width 0.6) (layer "B.Cu") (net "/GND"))
 (segment (start 61.75 61) (end 62 61) (width 0.6) (layer "B.Cu") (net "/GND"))
 (segment (start 60.5 62) (end 60.5 61.75) (width 0.6) (layer "B.Cu") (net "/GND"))
 (segment (start 66 55.75) (end 66.75 55.75) (width 0.6) (layer "B.Cu") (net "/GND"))
 (segment (start 76.5 47.5) (end 76.25 47.5) (width 0.6) (layer "B.Cu") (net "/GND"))
 (segment (start 76.25 47.5) (end 76.25 47.25) (width 0.6) (layer "B.Cu") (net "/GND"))
 (segment (start 62.5 60.5) (end 62.5 60.25) (width 0.6) (layer "B.Cu") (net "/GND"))
 (segment (start 77 48.75) (end 77 48) (width 0.6) (layer "B.Cu") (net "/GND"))
 (segment (start 45 65.5) (end 59 65.5) (width 0.6) (layer "B.Cu") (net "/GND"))
 (segment (start 68.25 54.75) (end 68.5 54.75) (width 0.6) (layer "B.Cu") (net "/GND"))
 (segment (start 59.75 62.25) (end 59.75 62) (width 0.6) (layer "B.Cu") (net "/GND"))
 (segment (start 29 66) (end 29 65.5) (width 0.6) (layer "B.Cu") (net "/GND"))
 (segment (start 63.25 58.75) (end 63.25 56) (width 0.6) (layer "B.Cu") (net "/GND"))
 (segment (start 59 62.25) (end 59.75 62.25) (width 0.6) (layer "B.Cu") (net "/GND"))
 (segment (start 61.5 61.25) (end 61.75 61.25) (width 0.6) (layer "B.Cu") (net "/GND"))
 (segment (start 76 47.25) (end 76 47) (width 0.6) (layer "B.Cu") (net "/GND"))
 (segment (start 76.5 53.75) (end 76.5 53.5) (width 0.6) (layer "B.Cu") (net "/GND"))
 (segment (start 75.75 54.25) (end 75.75 54) (width 0.6) (layer "B.Cu") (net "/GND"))
 (segment (start 59.75 62) (end 60.5 62) (width 0.6) (layer "B.Cu") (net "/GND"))
 (segment (start 75 54.5) (end 75 54.25) (width 0.6) (layer "B.Cu") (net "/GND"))
 (segment (start 61.25 61.75) (end 61.25 61.5) (width 0.6) (layer "B.Cu") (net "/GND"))
 (segment (start 76.75 53.5) (end 76.75 53) (width 0.6) (layer "B.Cu") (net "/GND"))
 (segment (start 76.75 48) (end 76.75 47.75) (width 0.6) (layer "B.Cu") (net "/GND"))
 (segment (start 75.5 26.5) (end 75.25 26.5) (width 0.6) (layer "B.Cu") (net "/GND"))
 (segment (start 59 65.5) (end 59 62.25) (width 0.6) (layer "B.Cu") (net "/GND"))
 (segment (start 66.75 55.5) (end 67.5 55.5) (width 0.6) (layer "B.Cu") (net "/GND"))
 (segment (start 77 53) (end 77 52.25) (width 0.6) (layer "B.Cu") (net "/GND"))
 (segment (start 68.5 54.75) (end 68.5 54.5) (width 0.6) (layer "B.Cu") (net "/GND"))
 (segment (start 67.5 55.25) (end 68 55.25) (width 0.6) (layer "B.Cu") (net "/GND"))
 (segment (start 77.25 48.75) (end 77 48.75) (width 0.6) (layer "B.Cu") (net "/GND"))
 (segment (start 60.5 61.75) (end 61.25 61.75) (width 0.6) (layer "B.Cu") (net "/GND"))
 (segment (start 77 52.25) (end 77.25 52.25) (width 0.6) (layer "B.Cu") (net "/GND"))
 (segment (start 8 12.5) (end 8 12.54) (width 0.6) (layer "B.Cu") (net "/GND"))
 (segment (start 75.25 26.5) (end 75.25 26.25) (width 0.6) (layer "B.Cu") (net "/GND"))
 (segment (start 75.5 47) (end 75.5 26.5) (width 0.6) (layer "B.Cu") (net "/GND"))
 (segment (start 76.25 53.75) (end 76.5 53.75) (width 0.6) (layer "B.Cu") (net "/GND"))
 (segment (start 75 26.25) (end 75 13) (width 0.6) (layer "B.Cu") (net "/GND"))
 (segment (start 61.75 61.25) (end 61.75 61) (width 0.6) (layer "B.Cu") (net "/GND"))
 (segment (start 59 65.5) (end 59 65.62) (width 0.6) (layer "B.Cu") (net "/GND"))
 (segment (start 62 60.75) (end 62.25 60.75) (width 0.6) (layer "B.Cu") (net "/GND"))
 (segment (start 61.25 61.5) (end 61.5 61.5) (width 0.6) (layer "B.Cu") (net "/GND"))
 (segment (start 77 48) (end 76.75 48) (width 0.6) (layer "B.Cu") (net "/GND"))
 (segment (start 63 59.5) (end 63 58.75) (width 0.6) (layer "B.Cu") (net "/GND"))
 (segment (start 61.5 61.5) (end 61.5 61.25) (width 0.6) (layer "B.Cu") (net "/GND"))
 (segment (start 75 54.25) (end 75.75 54.25) (width 0.6) (layer "B.Cu") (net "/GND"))
 (segment (start 62.25 60.75) (end 62.25 60.5) (width 0.6) (layer "B.Cu") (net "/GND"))
 (segment (start 76.25 54) (end 76.25 53.75) (width 0.6) (layer "B.Cu") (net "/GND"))
 (segment (start 45 65.62) (end 45 65.5) (width 0.6) (layer "B.Cu") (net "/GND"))
 (segment (start 66 56) (end 66 55.75) (width 0.6) (layer "B.Cu") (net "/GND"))
 (segment (start 8 66) (end 8 12.5) (width 0.6) (layer "B.Cu") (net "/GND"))
 (segment (start 76.75 53) (end 77 53) (width 0.6) (layer "B.Cu") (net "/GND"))
 (segment (start 77.25 52.25) (end 77.25 48.75) (width 0.6) (layer "B.Cu") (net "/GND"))
 (segment (start 29 58.38) (end 29 58.5) (width 0.6) (layer "B.Cu") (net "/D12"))
 (segment (start 29 58.5) (end 29 54) (width 0.6) (layer "B.Cu") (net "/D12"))
 (segment (start 45 50) (end 45 58) (width 0.6) (layer "B.Cu") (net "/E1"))
 (segment (start 40 50) (end 40 47.5) (width 0.6) (layer "B.Cu") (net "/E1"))
 (segment (start 45 50) (end 40 50) (width 0.6) (layer "B.Cu") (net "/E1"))
 (segment (start 40 47.5) (end 40 47.54) (width 0.6) (layer "B.Cu") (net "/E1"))
 (segment (start 29 46.38) (end 29 46.5) (width 0.6) (layer "B.Cu") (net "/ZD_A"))
 (segment (start 29 46.5) (end 29 42.5) (width 0.6) (layer "B.Cu") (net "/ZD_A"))
 (segment (start 29 42.5) (end 29 42.62) (width 0.6) (layer "B.Cu") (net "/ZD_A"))
 (segment (start 43 27.62) (end 43 27.5) (width 0.6) (layer "B.Cu") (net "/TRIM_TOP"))
 (segment (start 43 27.5) (end 43 38) (width 0.6) (layer "B.Cu") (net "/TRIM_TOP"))
 (segment (start 43 38) (end 45 38) (width 0.6) (layer "B.Cu") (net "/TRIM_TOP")))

